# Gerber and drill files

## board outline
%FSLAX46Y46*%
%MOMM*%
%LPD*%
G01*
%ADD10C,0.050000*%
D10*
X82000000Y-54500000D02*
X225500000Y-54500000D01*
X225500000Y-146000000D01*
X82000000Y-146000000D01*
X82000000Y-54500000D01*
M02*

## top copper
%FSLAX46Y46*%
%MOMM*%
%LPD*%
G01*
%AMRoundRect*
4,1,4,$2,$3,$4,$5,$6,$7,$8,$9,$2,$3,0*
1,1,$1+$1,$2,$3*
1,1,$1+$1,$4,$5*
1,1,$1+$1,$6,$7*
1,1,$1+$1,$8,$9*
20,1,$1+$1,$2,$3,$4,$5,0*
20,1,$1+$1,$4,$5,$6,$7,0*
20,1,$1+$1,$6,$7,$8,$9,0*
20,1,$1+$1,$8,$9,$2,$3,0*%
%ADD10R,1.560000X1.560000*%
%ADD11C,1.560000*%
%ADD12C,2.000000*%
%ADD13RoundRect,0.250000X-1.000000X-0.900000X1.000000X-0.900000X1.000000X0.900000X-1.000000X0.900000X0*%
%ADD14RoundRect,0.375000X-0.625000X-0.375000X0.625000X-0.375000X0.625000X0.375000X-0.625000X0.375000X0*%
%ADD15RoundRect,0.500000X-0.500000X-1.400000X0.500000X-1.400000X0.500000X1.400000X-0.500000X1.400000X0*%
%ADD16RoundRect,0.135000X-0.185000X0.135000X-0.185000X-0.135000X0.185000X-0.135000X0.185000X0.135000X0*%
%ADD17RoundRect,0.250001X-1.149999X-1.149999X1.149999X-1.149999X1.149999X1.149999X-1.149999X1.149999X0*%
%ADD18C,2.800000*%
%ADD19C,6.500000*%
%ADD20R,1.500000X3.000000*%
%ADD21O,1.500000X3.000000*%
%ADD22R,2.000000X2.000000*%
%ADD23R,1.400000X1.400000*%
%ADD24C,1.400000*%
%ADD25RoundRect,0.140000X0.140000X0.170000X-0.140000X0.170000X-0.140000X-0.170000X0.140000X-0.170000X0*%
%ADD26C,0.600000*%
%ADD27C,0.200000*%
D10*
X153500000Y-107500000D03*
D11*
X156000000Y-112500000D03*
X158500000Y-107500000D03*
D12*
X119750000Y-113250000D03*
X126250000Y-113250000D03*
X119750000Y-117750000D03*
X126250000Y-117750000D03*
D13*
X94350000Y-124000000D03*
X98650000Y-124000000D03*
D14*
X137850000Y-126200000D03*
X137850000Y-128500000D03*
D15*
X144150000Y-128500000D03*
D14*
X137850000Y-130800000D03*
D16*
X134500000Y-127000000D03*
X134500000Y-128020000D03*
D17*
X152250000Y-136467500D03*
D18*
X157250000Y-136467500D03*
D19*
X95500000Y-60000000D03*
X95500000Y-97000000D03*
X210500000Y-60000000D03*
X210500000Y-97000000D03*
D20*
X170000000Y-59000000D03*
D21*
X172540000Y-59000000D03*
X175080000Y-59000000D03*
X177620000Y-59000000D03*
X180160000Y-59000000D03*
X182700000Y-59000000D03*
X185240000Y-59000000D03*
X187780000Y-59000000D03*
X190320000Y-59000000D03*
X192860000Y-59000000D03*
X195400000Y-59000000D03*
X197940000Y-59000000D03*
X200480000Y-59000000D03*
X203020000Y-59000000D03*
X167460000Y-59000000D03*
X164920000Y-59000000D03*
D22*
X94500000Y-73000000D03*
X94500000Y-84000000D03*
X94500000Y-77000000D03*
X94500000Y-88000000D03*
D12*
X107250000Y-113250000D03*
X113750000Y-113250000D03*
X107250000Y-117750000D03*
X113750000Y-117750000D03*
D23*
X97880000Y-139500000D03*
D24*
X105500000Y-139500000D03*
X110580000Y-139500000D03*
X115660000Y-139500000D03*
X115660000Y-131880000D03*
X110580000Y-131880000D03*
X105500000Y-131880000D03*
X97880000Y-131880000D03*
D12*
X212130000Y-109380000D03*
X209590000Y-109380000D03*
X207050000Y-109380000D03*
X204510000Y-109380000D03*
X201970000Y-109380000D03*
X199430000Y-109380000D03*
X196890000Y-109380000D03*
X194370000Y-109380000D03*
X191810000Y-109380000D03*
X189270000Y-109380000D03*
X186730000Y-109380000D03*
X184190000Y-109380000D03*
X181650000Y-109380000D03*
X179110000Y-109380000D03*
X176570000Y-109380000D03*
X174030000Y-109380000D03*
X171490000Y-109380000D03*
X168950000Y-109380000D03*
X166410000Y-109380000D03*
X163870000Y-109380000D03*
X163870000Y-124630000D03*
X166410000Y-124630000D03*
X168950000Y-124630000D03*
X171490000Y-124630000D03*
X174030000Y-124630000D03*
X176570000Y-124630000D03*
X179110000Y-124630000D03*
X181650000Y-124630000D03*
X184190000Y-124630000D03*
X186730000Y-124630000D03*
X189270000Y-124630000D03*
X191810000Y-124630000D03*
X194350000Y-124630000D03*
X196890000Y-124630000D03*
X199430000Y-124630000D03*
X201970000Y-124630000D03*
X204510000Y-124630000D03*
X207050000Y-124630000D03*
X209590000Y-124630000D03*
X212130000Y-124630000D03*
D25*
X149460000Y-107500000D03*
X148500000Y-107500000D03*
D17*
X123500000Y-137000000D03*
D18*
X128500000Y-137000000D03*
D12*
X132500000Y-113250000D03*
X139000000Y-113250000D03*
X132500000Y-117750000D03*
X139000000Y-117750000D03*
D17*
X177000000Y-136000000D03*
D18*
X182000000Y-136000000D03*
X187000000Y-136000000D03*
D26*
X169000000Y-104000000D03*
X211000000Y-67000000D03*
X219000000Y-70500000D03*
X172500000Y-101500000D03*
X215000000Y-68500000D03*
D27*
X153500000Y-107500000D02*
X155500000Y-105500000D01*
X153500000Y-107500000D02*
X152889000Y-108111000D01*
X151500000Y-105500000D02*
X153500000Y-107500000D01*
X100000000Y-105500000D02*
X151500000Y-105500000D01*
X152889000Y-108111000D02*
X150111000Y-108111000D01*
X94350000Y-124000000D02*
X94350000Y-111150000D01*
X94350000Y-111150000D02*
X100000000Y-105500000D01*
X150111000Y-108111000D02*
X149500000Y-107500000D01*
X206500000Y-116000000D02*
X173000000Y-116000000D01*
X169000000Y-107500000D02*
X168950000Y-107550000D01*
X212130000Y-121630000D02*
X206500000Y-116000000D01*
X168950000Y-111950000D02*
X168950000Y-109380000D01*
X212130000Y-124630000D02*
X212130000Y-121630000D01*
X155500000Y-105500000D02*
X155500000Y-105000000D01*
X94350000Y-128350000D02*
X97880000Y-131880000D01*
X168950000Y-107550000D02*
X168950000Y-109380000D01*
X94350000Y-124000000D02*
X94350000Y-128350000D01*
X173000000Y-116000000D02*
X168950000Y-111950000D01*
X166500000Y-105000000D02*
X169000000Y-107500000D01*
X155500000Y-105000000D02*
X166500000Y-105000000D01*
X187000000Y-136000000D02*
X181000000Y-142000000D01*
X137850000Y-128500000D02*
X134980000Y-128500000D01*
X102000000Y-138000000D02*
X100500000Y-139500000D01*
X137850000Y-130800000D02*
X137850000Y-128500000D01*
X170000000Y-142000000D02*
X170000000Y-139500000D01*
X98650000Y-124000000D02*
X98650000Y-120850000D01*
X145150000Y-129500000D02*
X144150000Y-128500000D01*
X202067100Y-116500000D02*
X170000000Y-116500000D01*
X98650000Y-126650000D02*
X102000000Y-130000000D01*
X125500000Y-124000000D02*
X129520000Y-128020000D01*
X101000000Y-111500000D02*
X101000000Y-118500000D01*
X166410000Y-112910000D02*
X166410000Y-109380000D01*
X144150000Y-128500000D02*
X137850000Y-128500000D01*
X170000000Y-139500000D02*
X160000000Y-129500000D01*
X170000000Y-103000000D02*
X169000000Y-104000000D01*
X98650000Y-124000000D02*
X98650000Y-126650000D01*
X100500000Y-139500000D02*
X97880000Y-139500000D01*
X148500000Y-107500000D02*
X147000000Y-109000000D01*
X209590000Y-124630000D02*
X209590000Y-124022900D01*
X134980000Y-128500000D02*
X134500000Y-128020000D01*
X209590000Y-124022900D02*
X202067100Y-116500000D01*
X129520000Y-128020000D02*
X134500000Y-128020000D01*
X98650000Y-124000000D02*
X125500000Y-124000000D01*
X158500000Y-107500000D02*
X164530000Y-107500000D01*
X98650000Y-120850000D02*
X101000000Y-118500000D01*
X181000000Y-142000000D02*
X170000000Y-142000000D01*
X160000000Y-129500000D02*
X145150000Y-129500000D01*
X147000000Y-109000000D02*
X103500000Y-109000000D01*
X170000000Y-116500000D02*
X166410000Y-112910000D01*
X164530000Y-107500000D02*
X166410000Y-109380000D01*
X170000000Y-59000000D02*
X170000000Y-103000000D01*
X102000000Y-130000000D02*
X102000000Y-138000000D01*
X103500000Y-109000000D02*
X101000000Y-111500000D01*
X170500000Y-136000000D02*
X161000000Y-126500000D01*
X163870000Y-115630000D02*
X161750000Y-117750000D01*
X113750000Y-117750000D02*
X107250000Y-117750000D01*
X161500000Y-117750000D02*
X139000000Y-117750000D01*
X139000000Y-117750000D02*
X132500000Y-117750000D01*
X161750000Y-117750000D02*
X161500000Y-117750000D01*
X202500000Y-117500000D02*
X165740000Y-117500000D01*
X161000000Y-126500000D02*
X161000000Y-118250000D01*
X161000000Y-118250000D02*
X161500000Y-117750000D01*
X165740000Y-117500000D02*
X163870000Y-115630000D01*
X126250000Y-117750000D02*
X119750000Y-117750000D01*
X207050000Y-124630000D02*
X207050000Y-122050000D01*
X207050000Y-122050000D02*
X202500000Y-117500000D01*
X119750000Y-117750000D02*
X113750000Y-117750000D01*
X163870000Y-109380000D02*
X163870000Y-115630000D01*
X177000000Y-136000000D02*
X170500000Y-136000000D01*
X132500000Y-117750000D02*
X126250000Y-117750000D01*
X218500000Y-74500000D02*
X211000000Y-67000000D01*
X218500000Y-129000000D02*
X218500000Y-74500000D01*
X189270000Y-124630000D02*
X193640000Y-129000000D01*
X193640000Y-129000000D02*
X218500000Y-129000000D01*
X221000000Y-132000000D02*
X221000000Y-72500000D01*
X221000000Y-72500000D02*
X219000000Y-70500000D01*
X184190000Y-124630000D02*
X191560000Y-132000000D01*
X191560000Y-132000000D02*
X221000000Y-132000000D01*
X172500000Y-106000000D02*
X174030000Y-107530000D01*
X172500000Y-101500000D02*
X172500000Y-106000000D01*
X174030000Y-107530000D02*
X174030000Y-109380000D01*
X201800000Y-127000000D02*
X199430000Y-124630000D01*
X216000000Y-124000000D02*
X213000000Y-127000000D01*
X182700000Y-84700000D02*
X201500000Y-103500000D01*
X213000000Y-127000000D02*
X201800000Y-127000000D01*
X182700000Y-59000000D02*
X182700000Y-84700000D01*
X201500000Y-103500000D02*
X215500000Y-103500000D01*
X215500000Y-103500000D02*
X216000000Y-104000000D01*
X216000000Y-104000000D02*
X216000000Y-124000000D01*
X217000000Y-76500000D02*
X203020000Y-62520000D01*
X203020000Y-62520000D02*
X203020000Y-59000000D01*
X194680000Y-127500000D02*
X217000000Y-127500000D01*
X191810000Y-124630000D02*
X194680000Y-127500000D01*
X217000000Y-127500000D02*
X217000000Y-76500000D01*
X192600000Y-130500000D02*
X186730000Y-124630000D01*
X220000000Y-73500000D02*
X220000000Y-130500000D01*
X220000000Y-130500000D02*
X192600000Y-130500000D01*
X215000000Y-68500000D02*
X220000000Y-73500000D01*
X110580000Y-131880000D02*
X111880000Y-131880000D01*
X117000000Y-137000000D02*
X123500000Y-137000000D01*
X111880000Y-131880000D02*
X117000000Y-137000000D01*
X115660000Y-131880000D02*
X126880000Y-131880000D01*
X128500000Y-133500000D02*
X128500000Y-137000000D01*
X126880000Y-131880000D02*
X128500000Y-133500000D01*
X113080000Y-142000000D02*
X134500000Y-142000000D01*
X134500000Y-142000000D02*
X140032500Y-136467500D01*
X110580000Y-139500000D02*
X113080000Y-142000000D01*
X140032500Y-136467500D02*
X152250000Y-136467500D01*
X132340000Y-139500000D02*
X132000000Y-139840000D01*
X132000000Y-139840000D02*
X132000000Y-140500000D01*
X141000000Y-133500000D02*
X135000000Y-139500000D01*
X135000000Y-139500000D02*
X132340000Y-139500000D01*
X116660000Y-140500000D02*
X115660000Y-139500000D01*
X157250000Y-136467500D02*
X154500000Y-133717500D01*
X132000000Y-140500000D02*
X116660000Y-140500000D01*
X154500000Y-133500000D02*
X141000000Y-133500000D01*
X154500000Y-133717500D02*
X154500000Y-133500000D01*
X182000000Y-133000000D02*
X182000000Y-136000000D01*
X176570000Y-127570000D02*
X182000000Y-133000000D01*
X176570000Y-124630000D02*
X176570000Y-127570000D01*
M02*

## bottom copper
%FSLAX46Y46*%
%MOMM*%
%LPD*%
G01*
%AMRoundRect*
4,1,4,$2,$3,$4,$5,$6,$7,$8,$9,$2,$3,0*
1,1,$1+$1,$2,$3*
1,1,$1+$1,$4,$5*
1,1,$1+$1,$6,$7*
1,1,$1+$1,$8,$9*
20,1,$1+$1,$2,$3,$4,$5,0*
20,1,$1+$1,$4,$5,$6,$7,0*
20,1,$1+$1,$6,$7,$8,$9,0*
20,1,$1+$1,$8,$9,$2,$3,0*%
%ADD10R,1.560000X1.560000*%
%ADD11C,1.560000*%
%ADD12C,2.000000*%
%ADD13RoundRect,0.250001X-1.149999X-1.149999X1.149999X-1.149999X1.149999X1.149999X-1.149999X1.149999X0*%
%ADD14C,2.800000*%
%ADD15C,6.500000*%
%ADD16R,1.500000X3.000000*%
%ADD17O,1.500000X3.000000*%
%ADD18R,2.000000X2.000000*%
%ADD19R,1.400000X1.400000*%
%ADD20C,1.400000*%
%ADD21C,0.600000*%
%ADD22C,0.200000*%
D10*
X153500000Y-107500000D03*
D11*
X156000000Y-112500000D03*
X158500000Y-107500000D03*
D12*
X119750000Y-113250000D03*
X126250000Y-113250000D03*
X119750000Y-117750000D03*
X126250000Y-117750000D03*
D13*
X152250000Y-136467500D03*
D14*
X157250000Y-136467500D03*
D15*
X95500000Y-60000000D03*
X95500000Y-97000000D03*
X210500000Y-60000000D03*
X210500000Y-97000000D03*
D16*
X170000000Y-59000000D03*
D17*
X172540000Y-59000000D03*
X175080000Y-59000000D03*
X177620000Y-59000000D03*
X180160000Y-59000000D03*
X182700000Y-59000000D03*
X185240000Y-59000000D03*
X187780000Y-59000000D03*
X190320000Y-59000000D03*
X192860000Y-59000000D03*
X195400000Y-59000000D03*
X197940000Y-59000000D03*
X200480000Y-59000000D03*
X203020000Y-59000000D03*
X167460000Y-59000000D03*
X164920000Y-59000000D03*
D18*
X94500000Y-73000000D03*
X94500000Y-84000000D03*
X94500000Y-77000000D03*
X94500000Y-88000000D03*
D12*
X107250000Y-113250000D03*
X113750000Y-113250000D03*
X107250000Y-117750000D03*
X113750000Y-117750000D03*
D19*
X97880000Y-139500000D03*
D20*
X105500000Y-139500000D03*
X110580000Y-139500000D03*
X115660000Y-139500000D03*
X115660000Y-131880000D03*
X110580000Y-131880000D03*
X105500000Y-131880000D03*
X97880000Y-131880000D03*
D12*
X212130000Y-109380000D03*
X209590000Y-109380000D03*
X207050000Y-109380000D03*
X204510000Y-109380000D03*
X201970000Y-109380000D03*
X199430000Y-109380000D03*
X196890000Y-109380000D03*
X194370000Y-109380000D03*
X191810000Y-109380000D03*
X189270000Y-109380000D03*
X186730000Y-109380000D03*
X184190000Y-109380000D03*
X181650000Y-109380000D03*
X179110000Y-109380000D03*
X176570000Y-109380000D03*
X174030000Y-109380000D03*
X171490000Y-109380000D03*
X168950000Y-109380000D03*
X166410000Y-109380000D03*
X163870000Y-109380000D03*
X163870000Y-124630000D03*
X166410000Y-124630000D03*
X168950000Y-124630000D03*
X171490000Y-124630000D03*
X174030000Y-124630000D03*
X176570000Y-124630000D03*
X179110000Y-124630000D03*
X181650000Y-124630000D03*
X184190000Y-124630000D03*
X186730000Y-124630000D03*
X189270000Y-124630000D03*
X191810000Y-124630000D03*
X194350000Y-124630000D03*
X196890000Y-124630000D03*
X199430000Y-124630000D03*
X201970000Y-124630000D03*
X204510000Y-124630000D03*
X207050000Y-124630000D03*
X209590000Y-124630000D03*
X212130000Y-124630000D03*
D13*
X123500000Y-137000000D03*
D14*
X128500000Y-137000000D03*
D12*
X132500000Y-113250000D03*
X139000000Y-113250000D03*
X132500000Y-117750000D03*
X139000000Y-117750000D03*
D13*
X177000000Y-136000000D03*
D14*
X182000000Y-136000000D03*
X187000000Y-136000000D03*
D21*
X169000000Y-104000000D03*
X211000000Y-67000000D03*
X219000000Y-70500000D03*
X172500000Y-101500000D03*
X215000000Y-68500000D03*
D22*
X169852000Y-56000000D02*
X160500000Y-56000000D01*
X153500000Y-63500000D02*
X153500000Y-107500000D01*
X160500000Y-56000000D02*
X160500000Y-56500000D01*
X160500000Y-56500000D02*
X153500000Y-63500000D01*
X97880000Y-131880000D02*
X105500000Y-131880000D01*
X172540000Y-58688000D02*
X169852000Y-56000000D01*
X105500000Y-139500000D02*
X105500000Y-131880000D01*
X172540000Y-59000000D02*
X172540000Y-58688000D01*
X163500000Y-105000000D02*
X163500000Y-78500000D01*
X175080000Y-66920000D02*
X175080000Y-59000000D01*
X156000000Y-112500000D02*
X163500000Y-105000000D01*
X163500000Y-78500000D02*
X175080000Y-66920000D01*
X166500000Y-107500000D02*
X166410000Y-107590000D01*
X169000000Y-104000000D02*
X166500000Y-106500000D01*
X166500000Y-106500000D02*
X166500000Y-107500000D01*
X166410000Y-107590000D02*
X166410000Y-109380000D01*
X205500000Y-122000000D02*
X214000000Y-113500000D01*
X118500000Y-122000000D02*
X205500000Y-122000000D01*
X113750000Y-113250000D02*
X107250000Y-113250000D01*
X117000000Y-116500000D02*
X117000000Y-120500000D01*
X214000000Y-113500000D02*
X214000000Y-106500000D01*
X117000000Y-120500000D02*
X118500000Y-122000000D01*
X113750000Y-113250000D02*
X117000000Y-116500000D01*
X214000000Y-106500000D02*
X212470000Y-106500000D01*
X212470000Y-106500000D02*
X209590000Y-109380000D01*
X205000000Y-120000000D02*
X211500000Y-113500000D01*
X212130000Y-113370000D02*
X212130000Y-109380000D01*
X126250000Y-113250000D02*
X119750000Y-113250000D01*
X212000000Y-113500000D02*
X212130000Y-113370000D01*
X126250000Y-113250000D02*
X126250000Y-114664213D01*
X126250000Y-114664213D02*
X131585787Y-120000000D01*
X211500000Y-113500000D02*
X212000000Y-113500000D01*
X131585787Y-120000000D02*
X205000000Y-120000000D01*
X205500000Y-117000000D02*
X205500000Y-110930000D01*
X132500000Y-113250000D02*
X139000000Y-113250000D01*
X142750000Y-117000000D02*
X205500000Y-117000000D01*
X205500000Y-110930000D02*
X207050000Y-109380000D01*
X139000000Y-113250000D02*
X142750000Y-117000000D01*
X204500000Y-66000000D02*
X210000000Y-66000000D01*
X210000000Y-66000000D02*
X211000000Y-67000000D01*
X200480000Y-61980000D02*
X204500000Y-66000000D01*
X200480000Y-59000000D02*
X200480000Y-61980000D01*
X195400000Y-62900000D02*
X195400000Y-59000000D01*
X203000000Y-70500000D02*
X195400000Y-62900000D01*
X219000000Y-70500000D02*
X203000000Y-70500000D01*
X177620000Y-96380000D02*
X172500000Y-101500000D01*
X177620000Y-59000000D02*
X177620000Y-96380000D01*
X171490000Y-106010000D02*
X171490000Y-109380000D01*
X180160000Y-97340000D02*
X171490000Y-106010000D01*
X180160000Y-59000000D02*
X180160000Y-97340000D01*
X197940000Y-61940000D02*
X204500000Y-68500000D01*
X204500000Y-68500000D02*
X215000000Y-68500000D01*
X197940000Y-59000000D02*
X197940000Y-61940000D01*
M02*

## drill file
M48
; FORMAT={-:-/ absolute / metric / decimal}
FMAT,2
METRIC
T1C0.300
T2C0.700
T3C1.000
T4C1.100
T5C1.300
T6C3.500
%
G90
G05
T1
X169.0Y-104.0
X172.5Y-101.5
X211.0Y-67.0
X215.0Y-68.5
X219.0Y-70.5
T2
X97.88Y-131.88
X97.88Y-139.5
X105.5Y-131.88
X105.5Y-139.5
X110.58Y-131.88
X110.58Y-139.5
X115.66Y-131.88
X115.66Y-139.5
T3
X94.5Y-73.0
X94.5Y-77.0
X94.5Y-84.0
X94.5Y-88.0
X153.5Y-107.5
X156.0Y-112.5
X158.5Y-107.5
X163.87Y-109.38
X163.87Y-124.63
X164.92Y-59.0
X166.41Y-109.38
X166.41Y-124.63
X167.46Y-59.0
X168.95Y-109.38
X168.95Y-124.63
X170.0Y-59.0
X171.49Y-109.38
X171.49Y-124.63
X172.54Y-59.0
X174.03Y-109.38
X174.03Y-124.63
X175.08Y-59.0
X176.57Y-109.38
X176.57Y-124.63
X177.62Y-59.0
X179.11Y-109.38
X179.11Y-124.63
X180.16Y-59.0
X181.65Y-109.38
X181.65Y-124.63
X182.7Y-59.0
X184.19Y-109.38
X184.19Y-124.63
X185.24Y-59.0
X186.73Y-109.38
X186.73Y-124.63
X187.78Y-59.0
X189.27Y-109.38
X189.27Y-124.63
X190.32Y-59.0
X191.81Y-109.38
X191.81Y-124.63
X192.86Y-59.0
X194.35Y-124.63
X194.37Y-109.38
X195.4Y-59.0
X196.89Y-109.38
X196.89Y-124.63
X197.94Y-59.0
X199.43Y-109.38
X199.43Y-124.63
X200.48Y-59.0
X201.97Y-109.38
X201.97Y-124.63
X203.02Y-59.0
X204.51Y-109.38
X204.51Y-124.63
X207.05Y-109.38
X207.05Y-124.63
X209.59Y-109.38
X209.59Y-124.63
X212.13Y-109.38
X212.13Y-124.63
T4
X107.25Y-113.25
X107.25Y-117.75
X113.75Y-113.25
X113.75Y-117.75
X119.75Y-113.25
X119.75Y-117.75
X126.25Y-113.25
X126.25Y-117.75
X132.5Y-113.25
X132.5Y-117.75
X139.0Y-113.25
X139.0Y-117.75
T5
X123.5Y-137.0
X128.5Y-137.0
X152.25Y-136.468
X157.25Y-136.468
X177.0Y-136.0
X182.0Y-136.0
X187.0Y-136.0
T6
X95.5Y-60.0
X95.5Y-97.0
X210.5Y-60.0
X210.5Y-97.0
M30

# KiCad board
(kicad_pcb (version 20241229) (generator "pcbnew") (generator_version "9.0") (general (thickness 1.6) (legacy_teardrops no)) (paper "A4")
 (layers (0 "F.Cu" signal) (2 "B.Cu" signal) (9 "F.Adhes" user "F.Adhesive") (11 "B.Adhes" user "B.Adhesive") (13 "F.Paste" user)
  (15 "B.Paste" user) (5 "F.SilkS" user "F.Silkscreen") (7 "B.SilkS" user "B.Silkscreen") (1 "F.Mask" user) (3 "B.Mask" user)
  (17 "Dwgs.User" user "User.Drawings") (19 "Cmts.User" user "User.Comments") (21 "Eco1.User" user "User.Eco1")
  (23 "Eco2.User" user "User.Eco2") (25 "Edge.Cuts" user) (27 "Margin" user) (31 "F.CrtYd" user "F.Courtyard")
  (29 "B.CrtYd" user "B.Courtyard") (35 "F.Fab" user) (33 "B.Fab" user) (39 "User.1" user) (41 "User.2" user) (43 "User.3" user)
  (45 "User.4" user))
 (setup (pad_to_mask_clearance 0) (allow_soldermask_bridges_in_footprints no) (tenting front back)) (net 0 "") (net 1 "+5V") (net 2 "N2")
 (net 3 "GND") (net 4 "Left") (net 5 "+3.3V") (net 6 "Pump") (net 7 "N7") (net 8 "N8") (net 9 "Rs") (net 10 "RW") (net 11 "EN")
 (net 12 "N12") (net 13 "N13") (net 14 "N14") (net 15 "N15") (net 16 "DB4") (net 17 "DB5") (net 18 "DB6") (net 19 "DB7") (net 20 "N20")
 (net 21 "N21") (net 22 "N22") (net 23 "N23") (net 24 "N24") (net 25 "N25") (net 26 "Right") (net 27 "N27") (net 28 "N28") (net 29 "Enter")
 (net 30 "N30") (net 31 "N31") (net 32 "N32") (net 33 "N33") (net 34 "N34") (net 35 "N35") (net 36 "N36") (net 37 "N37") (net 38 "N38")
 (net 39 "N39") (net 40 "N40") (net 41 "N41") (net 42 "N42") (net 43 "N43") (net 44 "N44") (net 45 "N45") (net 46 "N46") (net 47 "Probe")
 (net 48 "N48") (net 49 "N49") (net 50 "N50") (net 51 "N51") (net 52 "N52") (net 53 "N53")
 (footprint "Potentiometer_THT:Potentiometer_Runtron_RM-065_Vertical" (layer "F.Cu") (at 153.5 107.5)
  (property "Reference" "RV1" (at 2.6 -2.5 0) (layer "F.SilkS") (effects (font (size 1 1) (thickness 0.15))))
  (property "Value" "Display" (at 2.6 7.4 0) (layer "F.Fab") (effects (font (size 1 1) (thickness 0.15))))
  (pad "1" thru_hole rect (at 0 0) (size 1.56 1.56) (drill 1) (layers "*.Cu" "*.Mask") (remove_unused_layers no) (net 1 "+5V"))
  (pad "2" thru_hole circle (at 2.5 5) (size 1.56 1.56) (drill 1) (layers "*.Cu" "*.Mask") (remove_unused_layers no) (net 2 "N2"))
  (pad "3" thru_hole circle (at 5 0) (size 1.56 1.56) (drill 1) (layers "*.Cu" "*.Mask") (remove_unused_layers no) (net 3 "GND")))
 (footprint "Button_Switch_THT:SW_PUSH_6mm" (layer "F.Cu") (at 119.75 113.25)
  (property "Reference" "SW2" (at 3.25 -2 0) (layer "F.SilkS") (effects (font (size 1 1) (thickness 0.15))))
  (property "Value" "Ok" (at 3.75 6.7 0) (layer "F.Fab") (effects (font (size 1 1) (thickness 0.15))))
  (pad "1" thru_hole circle (at 0 0 90) (size 2 2) (drill 1.1) (layers "*.Cu" "*.Mask") (remove_unused_layers no) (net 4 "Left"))
  (pad "1" thru_hole circle (at 6.5 0 90) (size 2 2) (drill 1.1) (layers "*.Cu" "*.Mask") (remove_unused_layers no) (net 4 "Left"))
  (pad "2" thru_hole circle (at 0 4.5 90) (size 2 2) (drill 1.1) (layers "*.Cu" "*.Mask") (remove_unused_layers no) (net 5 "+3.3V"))
  (pad "2" thru_hole circle (at 6.5 4.5 90) (size 2 2) (drill 1.1) (layers "*.Cu" "*.Mask") (remove_unused_layers no) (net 5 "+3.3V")))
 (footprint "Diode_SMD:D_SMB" (layer "F.Cu") (at 96.5 124)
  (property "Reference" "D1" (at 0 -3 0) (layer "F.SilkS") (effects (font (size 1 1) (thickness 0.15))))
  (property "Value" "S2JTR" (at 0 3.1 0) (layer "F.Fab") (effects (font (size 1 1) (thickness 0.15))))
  (pad "1" smd roundrect (at -2.15 0) (size 2.5 2.3) (layers "F.Cu" "F.Mask" "F.Paste") (roundrect_rratio 0.1086956522) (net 1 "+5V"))
  (pad "2" smd roundrect (at 2.15 0) (size 2.5 2.3) (layers "F.Cu" "F.Mask" "F.Paste") (roundrect_rratio 0.1086956522) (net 3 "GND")))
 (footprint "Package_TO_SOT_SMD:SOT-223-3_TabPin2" (layer "F.Cu") (at 141 128.5)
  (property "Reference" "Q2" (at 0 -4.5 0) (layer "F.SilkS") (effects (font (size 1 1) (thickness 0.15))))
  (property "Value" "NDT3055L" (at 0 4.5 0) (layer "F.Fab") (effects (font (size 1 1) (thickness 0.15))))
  (pad "1" smd roundrect (at -3.15 -2.3) (size 2 1.5) (layers "F.Cu" "F.Mask" "F.Paste") (roundrect_rratio 0.25) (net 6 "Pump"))
  (pad "2" smd roundrect (at -3.15 0) (size 2 1.5) (layers "F.Cu" "F.Mask" "F.Paste") (roundrect_rratio 0.25) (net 3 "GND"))
  (pad "2" smd roundrect (at 3.15 0) (size 2 3.8) (layers "F.Cu" "F.Mask" "F.Paste") (roundrect_rratio 0.25) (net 3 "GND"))
  (pad "3" smd roundrect (at -3.15 2.3) (size 2 1.5) (layers "F.Cu" "F.Mask" "F.Paste") (roundrect_rratio 0.25) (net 3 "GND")))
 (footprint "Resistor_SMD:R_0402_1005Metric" (layer "F.Cu") (at 134.5 127.51 -90)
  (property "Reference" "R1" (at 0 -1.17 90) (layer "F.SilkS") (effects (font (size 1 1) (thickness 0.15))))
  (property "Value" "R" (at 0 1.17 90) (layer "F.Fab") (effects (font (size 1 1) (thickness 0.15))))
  (pad "1" smd roundrect (at -0.51 0 270) (size 0.54 0.64) (layers "F.Cu" "F.Mask" "F.Paste") (roundrect_rratio 0.25) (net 6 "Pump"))
  (pad "2" smd roundrect (at 0.51 0 270) (size 0.54 0.64) (layers "F.Cu" "F.Mask" "F.Paste") (roundrect_rratio 0.25) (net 3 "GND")))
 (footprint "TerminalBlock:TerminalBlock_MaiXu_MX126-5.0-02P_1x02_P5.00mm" (layer "F.Cu") (at 152.25 136.4675)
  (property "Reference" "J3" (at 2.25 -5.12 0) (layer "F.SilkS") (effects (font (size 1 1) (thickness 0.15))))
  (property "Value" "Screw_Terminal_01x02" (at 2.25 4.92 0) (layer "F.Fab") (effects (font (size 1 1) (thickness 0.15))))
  (pad "1" thru_hole roundrect (at 0 0) (size 2.8 2.8) (drill 1.3) (layers "*.Cu" "*.Mask") (remove_unused_layers no)
   (roundrect_rratio 0.089286) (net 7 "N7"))
  (pad "2" thru_hole circle (at 5 0) (size 2.8 2.8) (drill 1.3) (layers "*.Cu" "*.Mask") (remove_unused_layers no) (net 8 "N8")))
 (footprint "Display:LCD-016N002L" (layer "F.Cu") (at 170 59)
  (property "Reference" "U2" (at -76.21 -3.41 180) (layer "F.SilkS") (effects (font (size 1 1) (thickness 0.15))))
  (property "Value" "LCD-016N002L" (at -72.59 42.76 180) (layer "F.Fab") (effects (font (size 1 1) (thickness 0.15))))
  (pad "" thru_hole circle (at -74.5 1 180) (size 6.5 6.5) (drill 3.5) (layers "*.Cu" "*.Mask") (remove_unused_layers no))
  (pad "" thru_hole circle (at -74.5 38 180) (size 6.5 6.5) (drill 3.5) (layers "*.Cu" "*.Mask") (remove_unused_layers no))
  (pad "" thru_hole circle (at 40.5 1 180) (size 6.5 6.5) (drill 3.5) (layers "*.Cu" "*.Mask") (remove_unused_layers no))
  (pad "" thru_hole circle (at 40.5 38 180) (size 6.5 6.5) (drill 3.5) (layers "*.Cu" "*.Mask") (remove_unused_layers no))
  (pad "1" thru_hole rect (at 0 0 180) (size 1.5 3) (drill 1) (layers "*.Cu" "*.Mask") (remove_unused_layers no) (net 3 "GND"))
  (pad "2" thru_hole oval (at 2.54 0 180) (size 1.5 3) (drill 1) (layers "*.Cu" "*.Mask") (remove_unused_layers no) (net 1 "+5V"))
  (pad "3" thru_hole oval (at 5.08 0 180) (size 1.5 3) (drill 1) (layers "*.Cu" "*.Mask") (remove_unused_layers no) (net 2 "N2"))
  (pad "4" thru_hole oval (at 7.62 0 180) (size 1.5 3) (drill 1) (layers "*.Cu" "*.Mask") (remove_unused_layers no) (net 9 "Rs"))
  (pad "5" thru_hole oval (at 10.16 0 180) (size 1.5 3) (drill 1) (layers "*.Cu" "*.Mask") (remove_unused_layers no) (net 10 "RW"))
  (pad "6" thru_hole oval (at 12.7 0 180) (size 1.5 3) (drill 1) (layers "*.Cu" "*.Mask") (remove_unused_layers no) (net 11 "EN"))
  (pad "7" thru_hole oval (at 15.24 0 180) (size 1.5 3) (drill 1) (layers "*.Cu" "*.Mask") (remove_unused_layers no) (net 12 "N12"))
  (pad "8" thru_hole oval (at 17.78 0 180) (size 1.5 3) (drill 1) (layers "*.Cu" "*.Mask") (remove_unused_layers no) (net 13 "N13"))
  (pad "9" thru_hole oval (at 20.32 0 180) (size 1.5 3) (drill 1) (layers "*.Cu" "*.Mask") (remove_unused_layers no) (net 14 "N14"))
  (pad "10" thru_hole oval (at 22.86 0 180) (size 1.5 3) (drill 1) (layers "*.Cu" "*.Mask") (remove_unused_layers no) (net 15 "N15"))
  (pad "11" thru_hole oval (at 25.4 0 180) (size 1.5 3) (drill 1) (layers "*.Cu" "*.Mask") (remove_unused_layers no) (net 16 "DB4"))
  (pad "12" thru_hole oval (at 27.94 0 180) (size 1.5 3) (drill 1) (layers "*.Cu" "*.Mask") (remove_unused_layers no) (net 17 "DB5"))
  (pad "13" thru_hole oval (at 30.48 0 180) (size 1.5 3) (drill 1) (layers "*.Cu" "*.Mask") (remove_unused_layers no) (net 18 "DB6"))
  (pad "14" thru_hole oval (at 33.02 0 180) (size 1.5 3) (drill 1) (layers "*.Cu" "*.Mask") (remove_unused_layers no) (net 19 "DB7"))
  (pad "15" thru_hole oval (at -2.54 0 180) (size 1.5 3) (drill 1) (layers "*.Cu" "*.Mask") (remove_unused_layers no) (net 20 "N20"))
  (pad "16" thru_hole oval (at -5.08 0 180) (size 1.5 3) (drill 1) (layers "*.Cu" "*.Mask") (remove_unused_layers no) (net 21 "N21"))
  (pad "A1" thru_hole rect (at -75.5 14 180) (size 2 2) (drill 1) (layers "*.Cu" "*.Mask") (remove_unused_layers no) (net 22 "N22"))
  (pad "A2" thru_hole rect (at -75.5 25 180) (size 2 2) (drill 1) (layers "*.Cu" "*.Mask") (remove_unused_layers no) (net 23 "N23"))
  (pad "K1" thru_hole rect (at -75.5 18 180) (size 2 2) (drill 1) (layers "*.Cu" "*.Mask") (remove_unused_layers no) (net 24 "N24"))
  (pad "K2" thru_hole rect (at -75.5 29 180) (size 2 2) (drill 1) (layers "*.Cu" "*.Mask") (remove_unused_layers no) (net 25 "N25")))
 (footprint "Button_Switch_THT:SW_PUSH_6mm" (layer "F.Cu") (at 107.25 113.25)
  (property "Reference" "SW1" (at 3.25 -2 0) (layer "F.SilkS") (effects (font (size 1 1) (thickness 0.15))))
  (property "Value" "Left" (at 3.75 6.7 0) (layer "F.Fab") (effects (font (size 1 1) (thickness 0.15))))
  (pad "1" thru_hole circle (at 0 0 90) (size 2 2) (drill 1.1) (layers "*.Cu" "*.Mask") (remove_unused_layers no) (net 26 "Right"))
  (pad "1" thru_hole circle (at 6.5 0 90) (size 2 2) (drill 1.1) (layers "*.Cu" "*.Mask") (remove_unused_layers no) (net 26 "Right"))
  (pad "2" thru_hole circle (at 0 4.5 90) (size 2 2) (drill 1.1) (layers "*.Cu" "*.Mask") (remove_unused_layers no) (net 5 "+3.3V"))
  (pad "2" thru_hole circle (at 6.5 4.5 90) (size 2 2) (drill 1.1) (layers "*.Cu" "*.Mask") (remove_unused_layers no) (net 5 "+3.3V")))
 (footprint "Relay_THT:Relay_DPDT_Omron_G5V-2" (layer "F.Cu") (at 97.88 139.5 90)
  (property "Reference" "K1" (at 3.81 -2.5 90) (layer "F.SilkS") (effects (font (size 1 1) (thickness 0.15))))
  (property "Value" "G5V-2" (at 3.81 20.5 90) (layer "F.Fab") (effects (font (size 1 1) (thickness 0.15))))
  (pad "1" thru_hole rect (at 0 0 90) (size 1.4 1.4) (drill 0.7) (layers "*.Cu" "*.Mask") (remove_unused_layers no) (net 3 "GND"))
  (pad "4" thru_hole circle (at 0 7.62 90) (size 1.4 1.4) (drill 0.7) (layers "*.Cu" "*.Mask") (remove_unused_layers no) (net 1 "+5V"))
  (pad "6" thru_hole circle (at 0 12.7 90) (size 1.4 1.4) (drill 0.7) (layers "*.Cu" "*.Mask") (remove_unused_layers no) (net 7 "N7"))
  (pad "8" thru_hole circle (at 0 17.78 90) (size 1.4 1.4) (drill 0.7) (layers "*.Cu" "*.Mask") (remove_unused_layers no) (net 8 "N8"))
  (pad "9" thru_hole circle (at 7.62 17.78 90) (size 1.4 1.4) (drill 0.7) (layers "*.Cu" "*.Mask") (remove_unused_layers no) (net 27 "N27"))
  (pad "11" thru_hole circle (at 7.62 12.7 90) (size 1.4 1.4) (drill 0.7) (layers "*.Cu" "*.Mask") (remove_unused_layers no) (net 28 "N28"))
  (pad "13" thru_hole circle (at 7.62 7.62 90) (size 1.4 1.4) (drill 0.7) (layers "*.Cu" "*.Mask") (remove_unused_layers no) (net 1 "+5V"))
  (pad "16" thru_hole circle (at 7.62 0 90) (size 1.4 1.4) (drill 0.7) (layers "*.Cu" "*.Mask") (remove_unused_layers no) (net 1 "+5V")))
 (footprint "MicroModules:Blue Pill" (layer "F.Cu") (at 212.13 109.38 90)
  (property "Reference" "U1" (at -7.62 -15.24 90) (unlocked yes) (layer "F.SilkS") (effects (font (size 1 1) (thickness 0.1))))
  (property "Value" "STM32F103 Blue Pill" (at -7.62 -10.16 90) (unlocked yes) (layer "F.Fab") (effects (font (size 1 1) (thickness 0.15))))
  (pad "1" thru_hole circle (at 0 0 90) (size 2 2) (drill 1) (layers "*.Cu" "*.Mask") (remove_unused_layers no) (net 4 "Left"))
  (pad "2" thru_hole circle (at 0 -2.54 90) (size 2 2) (drill 1) (layers "*.Cu" "*.Mask") (remove_unused_layers no) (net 26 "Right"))
  (pad "3" thru_hole circle (at 0 -5.08 90) (size 2 2) (drill 1) (layers "*.Cu" "*.Mask") (remove_unused_layers no) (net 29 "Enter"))
  (pad "4" thru_hole circle (at 0 -7.62 90) (size 2 2) (drill 1) (layers "*.Cu" "*.Mask") (remove_unused_layers no) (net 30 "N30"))
  (pad "5" thru_hole circle (at 0 -10.16 90) (size 2 2) (drill 1) (layers "*.Cu" "*.Mask") (remove_unused_layers no) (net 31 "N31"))
  (pad "6" thru_hole circle (at 0 -12.7 90) (size 2 2) (drill 1) (layers "*.Cu" "*.Mask") (remove_unused_layers no) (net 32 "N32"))
  (pad "7" thru_hole circle (at 0 -15.24 90) (size 2 2) (drill 1) (layers "*.Cu" "*.Mask") (remove_unused_layers no) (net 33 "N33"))
  (pad "8" thru_hole circle (at 0 -17.76 90) (size 2 2) (drill 1) (layers "*.Cu" "*.Mask") (remove_unused_layers no) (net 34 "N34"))
  (pad "9" thru_hole circle (at 0 -20.32 90) (size 2 2) (drill 1) (layers "*.Cu" "*.Mask") (remove_unused_layers no) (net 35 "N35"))
  (pad "10" thru_hole circle (at 0 -22.86 90) (size 2 2) (drill 1) (layers "*.Cu" "*.Mask") (remove_unused_layers no) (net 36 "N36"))
  (pad "11" thru_hole circle (at 0 -25.4 90) (size 2 2) (drill 1) (layers "*.Cu" "*.Mask") (remove_unused_layers no) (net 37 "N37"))
  (pad "12" thru_hole circle (at 0 -27.94 90) (size 2 2) (drill 1) (layers "*.Cu" "*.Mask") (remove_unused_layers no) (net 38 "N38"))
  (pad "13" thru_hole circle (at 0 -30.48 90) (size 2 2) (drill 1) (layers "*.Cu" "*.Mask") (remove_unused_layers no) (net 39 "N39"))
  (pad "14" thru_hole circle (at 0 -33.02 90) (size 2 2) (drill 1) (layers "*.Cu" "*.Mask") (remove_unused_layers no) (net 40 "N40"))
  (pad "15" thru_hole circle (at 0 -35.56 90) (size 2 2) (drill 1) (layers "*.Cu" "*.Mask") (remove_unused_layers no) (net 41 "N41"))
  (pad "16" thru_hole circle (at 0 -38.1 90) (size 2 2) (drill 1) (layers "*.Cu" "*.Mask") (remove_unused_layers no) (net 9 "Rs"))
  (pad "17" thru_hole circle (at 0 -40.64 90) (size 2 2) (drill 1) (layers "*.Cu" "*.Mask") (remove_unused_layers no) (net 10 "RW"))
  (pad "18" thru_hole circle (at 0 -43.18 90) (size 2 2) (drill 1) (layers "*.Cu" "*.Mask") (remove_unused_layers no) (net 1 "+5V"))
  (pad "19" thru_hole circle (at 0 -45.72 90) (size 2 2) (drill 1) (layers "*.Cu" "*.Mask") (remove_unused_layers no) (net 3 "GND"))
  (pad "20" thru_hole circle (at 0 -48.26 90) (size 2 2) (drill 1) (layers "*.Cu" "*.Mask") (remove_unused_layers no) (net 5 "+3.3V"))
  (pad "21" thru_hole circle (at -15.25 -48.26 90) (size 2 2) (drill 1) (layers "*.Cu" "*.Mask") (remove_unused_layers no) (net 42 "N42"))
  (pad "22" thru_hole circle (at -15.25 -45.72 90) (size 2 2) (drill 1) (layers "*.Cu" "*.Mask") (remove_unused_layers no) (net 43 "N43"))
  (pad "23" thru_hole circle (at -15.25 -43.18 90) (size 2 2) (drill 1) (layers "*.Cu" "*.Mask") (remove_unused_layers no) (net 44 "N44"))
  (pad "24" thru_hole circle (at -15.25 -40.64 90) (size 2 2) (drill 1) (layers "*.Cu" "*.Mask") (remove_unused_layers no) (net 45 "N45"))
  (pad "25" thru_hole circle (at -15.25 -38.1 90) (size 2 2) (drill 1) (layers "*.Cu" "*.Mask") (remove_unused_layers no) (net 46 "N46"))
  (pad "26" thru_hole circle (at -15.25 -35.56 90) (size 2 2) (drill 1) (layers "*.Cu" "*.Mask") (remove_unused_layers no) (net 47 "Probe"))
  (pad "27" thru_hole circle (at -15.25 -33.02 90) (size 2 2) (drill 1) (layers "*.Cu" "*.Mask") (remove_unused_layers no) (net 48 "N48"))
  (pad "28" thru_hole circle (at -15.25 -30.48 90) (size 2 2) (drill 1) (layers "*.Cu" "*.Mask") (remove_unused_layers no) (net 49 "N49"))
  (pad "29" thru_hole circle (at -15.25 -27.94 90) (size 2 2) (drill 1) (layers "*.Cu" "*.Mask") (remove_unused_layers no) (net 16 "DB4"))
  (pad "30" thru_hole circle (at -15.25 -25.4 90) (size 2 2) (drill 1) (layers "*.Cu" "*.Mask") (remove_unused_layers no) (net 17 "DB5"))
  (pad "31" thru_hole circle (at -15.25 -22.86 90) (size 2 2) (drill 1) (layers "*.Cu" "*.Mask") (remove_unused_layers no) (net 18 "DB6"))
  (pad "32" thru_hole circle (at -15.25 -20.32 90) (size 2 2) (drill 1) (layers "*.Cu" "*.Mask") (remove_unused_layers no) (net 19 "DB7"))
  (pad "33" thru_hole circle (at -15.25 -17.78 90) (size 2 2) (drill 1) (layers "*.Cu" "*.Mask") (remove_unused_layers no) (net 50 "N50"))
  (pad "34" thru_hole circle (at -15.25 -15.24 90) (size 2 2) (drill 1) (layers "*.Cu" "*.Mask") (remove_unused_layers no) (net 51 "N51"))
  (pad "35" thru_hole circle (at -15.25 -12.7 90) (size 2 2) (drill 1) (layers "*.Cu" "*.Mask") (remove_unused_layers no) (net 11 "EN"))
  (pad "36" thru_hole circle (at -15.25 -10.16 90) (size 2 2) (drill 1) (layers "*.Cu" "*.Mask") (remove_unused_layers no) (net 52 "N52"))
  (pad "37" thru_hole circle (at -15.25 -7.62 90) (size 2 2) (drill 1) (layers "*.Cu" "*.Mask") (remove_unused_layers no) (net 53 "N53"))
  (pad "38" thru_hole circle (at -15.25 -5.08 90) (size 2 2) (drill 1) (layers "*.Cu" "*.Mask") (remove_unused_layers no) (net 5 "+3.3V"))
  (pad "39" thru_hole circle (at -15.25 -2.54 90) (size 2 2) (drill 1) (layers "*.Cu" "*.Mask") (remove_unused_layers no) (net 3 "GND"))
  (pad "40" thru_hole circle (at -15.25 0 90) (size 2 2) (drill 1) (layers "*.Cu" "*.Mask") (remove_unused_layers no) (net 1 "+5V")))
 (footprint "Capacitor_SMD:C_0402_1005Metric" (layer "F.Cu") (at 148.98 107.5 180)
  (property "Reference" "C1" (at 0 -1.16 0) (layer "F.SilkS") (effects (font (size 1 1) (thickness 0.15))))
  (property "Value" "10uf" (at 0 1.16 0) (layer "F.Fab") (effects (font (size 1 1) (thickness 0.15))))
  (pad "1" smd roundrect (at -0.48 0 180) (size 0.56 0.62) (layers "F.Cu" "F.Mask" "F.Paste") (roundrect_rratio 0.25) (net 1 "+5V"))
  (pad "2" smd roundrect (at 0.48 0 180) (size 0.56 0.62) (layers "F.Cu" "F.Mask" "F.Paste") (roundrect_rratio 0.25) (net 3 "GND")))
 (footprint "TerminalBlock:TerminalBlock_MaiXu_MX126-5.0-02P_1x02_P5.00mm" (layer "F.Cu") (at 123.5 137)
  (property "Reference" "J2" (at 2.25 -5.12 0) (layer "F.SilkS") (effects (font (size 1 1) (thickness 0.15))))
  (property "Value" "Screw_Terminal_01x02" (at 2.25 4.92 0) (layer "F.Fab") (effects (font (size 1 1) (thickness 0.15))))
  (pad "1" thru_hole roundrect (at 0 0) (size 2.8 2.8) (drill 1.3) (layers "*.Cu" "*.Mask") (remove_unused_layers no)
   (roundrect_rratio 0.089286) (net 28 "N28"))
  (pad "2" thru_hole circle (at 5 0) (size 2.8 2.8) (drill 1.3) (layers "*.Cu" "*.Mask") (remove_unused_layers no) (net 27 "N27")))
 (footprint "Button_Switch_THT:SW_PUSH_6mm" (layer "F.Cu") (at 132.5 113.25)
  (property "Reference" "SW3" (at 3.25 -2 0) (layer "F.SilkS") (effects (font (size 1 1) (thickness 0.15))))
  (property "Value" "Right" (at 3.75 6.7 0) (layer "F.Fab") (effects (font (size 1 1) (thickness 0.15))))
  (pad "1" thru_hole circle (at 0 0 90) (size 2 2) (drill 1.1) (layers "*.Cu" "*.Mask") (remove_unused_layers no) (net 29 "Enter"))
  (pad "1" thru_hole circle (at 6.5 0 90) (size 2 2) (drill 1.1) (layers "*.Cu" "*.Mask") (remove_unused_layers no) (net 29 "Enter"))
  (pad "2" thru_hole circle (at 0 4.5 90) (size 2 2) (drill 1.1) (layers "*.Cu" "*.Mask") (remove_unused_layers no) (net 5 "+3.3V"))
  (pad "2" thru_hole circle (at 6.5 4.5 90) (size 2 2) (drill 1.1) (layers "*.Cu" "*.Mask") (remove_unused_layers no) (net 5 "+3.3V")))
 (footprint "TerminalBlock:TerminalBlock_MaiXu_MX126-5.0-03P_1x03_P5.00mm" (layer "F.Cu") (at 177 136)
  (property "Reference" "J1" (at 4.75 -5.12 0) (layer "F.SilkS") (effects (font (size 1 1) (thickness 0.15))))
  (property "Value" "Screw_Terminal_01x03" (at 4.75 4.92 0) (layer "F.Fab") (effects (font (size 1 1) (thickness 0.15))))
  (pad "1" thru_hole roundrect (at 0 0) (size 2.8 2.8) (drill 1.3) (layers "*.Cu" "*.Mask") (remove_unused_layers no)
   (roundrect_rratio 0.089286) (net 5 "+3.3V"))
  (pad "2" thru_hole circle (at 5 0) (size 2.8 2.8) (drill 1.3) (layers "*.Cu" "*.Mask") (remove_unused_layers no) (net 47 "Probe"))
  (pad "3" thru_hole circle (at 10 0) (size 2.8 2.8) (drill 1.3) (layers "*.Cu" "*.Mask") (remove_unused_layers no) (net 3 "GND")))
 (gr_rect (start 82 54.5) (end 225.5 146) (stroke (width 0.05) (type default)) (fill no) (layer "Edge.Cuts"))
 (segment (start 153.5 107.5) (end 155.5 105.5) (width 0.2) (layer "F.Cu") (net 1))
 (segment (start 153.5 107.5) (end 152.889 108.111) (width 0.2) (layer "F.Cu") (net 1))
 (segment (start 151.5 105.5) (end 153.5 107.5) (width 0.2) (layer "F.Cu") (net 1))
 (segment (start 100 105.5) (end 151.5 105.5) (width 0.2) (layer "F.Cu") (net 1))
 (segment (start 152.889 108.111) (end 150.111 108.111) (width 0.2) (layer "F.Cu") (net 1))
 (segment (start 94.35 124) (end 94.35 111.15) (width 0.2) (layer "F.Cu") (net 1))
 (segment (start 94.35 111.15) (end 100 105.5) (width 0.2) (layer "F.Cu") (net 1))
 (segment (start 150.111 108.111) (end 149.5 107.5) (width 0.2) (layer "F.Cu") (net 1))
 (segment (start 206.5 116) (end 173 116) (width 0.2) (layer "F.Cu") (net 1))
 (segment (start 169 107.5) (end 168.95 107.55) (width 0.2) (layer "F.Cu") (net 1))
 (segment (start 212.13 121.63) (end 206.5 116) (width 0.2) (layer "F.Cu") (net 1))
 (segment (start 168.95 111.95) (end 168.95 109.38) (width 0.2) (layer "F.Cu") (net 1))
 (segment (start 212.13 124.63) (end 212.13 121.63) (width 0.2) (layer "F.Cu") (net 1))
 (segment (start 155.5 105.5) (end 155.5 105) (width 0.2) (layer "F.Cu") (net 1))
 (segment (start 94.35 128.35) (end 97.88 131.88) (width 0.2) (layer "F.Cu") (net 1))
 (segment (start 168.95 107.55) (end 168.95 109.38) (width 0.2) (layer "F.Cu") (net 1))
 (segment (start 94.35 124) (end 94.35 128.35) (width 0.2) (layer "F.Cu") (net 1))
 (segment (start 173 116) (end 168.95 111.95) (width 0.2) (layer "F.Cu") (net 1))
 (segment (start 166.5 105) (end 169 107.5) (width 0.2) (layer "F.Cu") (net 1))
 (segment (start 155.5 105) (end 166.5 105) (width 0.2) (layer "F.Cu") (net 1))
 (segment (start 169.852 56) (end 160.5 56) (width 0.2) (layer "B.Cu") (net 1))
 (segment (start 153.5 63.5) (end 153.5 107.5) (width 0.2) (layer "B.Cu") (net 1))
 (segment (start 160.5 56) (end 160.5 56.5) (width 0.2) (layer "B.Cu") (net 1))
 (segment (start 160.5 56.5) (end 153.5 63.5) (width 0.2) (layer "B.Cu") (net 1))
 (segment (start 97.88 131.88) (end 105.5 131.88) (width 0.2) (layer "B.Cu") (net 1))
 (segment (start 172.54 58.688) (end 169.852 56) (width 0.2) (layer "B.Cu") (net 1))
 (segment (start 105.5 139.5) (end 105.5 131.88) (width 0.2) (layer "B.Cu") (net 1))
 (segment (start 172.54 59) (end 172.54 58.688) (width 0.2) (layer "B.Cu") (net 1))
 (segment (start 163.5 105) (end 163.5 78.5) (width 0.2) (layer "B.Cu") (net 2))
 (segment (start 175.08 66.92) (end 175.08 59) (width 0.2) (layer "B.Cu") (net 2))
 (segment (start 156 112.5) (end 163.5 105) (width 0.2) (layer "B.Cu") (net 2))
 (segment (start 163.5 78.5) (end 175.08 66.92) (width 0.2) (layer "B.Cu") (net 2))
 (segment (start 187 136) (end 181 142) (width 0.2) (layer "F.Cu") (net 3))
 (segment (start 137.85 128.5) (end 134.98 128.5) (width 0.2) (layer "F.Cu") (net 3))
 (segment (start 102 138) (end 100.5 139.5) (width 0.2) (layer "F.Cu") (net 3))
 (segment (start 137.85 130.8) (end 137.85 128.5) (width 0.2) (layer "F.Cu") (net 3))
 (segment (start 170 142) (end 170 139.5) (width 0.2) (layer "F.Cu") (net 3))
 (segment (start 98.65 124) (end 98.65 120.85) (width 0.2) (layer "F.Cu") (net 3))
 (segment (start 145.15 129.5) (end 144.15 128.5) (width 0.2) (layer "F.Cu") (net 3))
 (segment (start 202.0671 116.5) (end 170 116.5) (width 0.2) (layer "F.Cu") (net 3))
 (segment (start 98.65 126.65) (end 102 130) (width 0.2) (layer "F.Cu") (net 3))
 (segment (start 125.5 124) (end 129.52 128.02) (width 0.2) (layer "F.Cu") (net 3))
 (segment (start 101 111.5) (end 101 118.5) (width 0.2) (layer "F.Cu") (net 3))
 (segment (start 166.41 112.91) (end 166.41 109.38) (width 0.2) (layer "F.Cu") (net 3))
 (segment (start 144.15 128.5) (end 137.85 128.5) (width 0.2) (layer "F.Cu") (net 3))
 (segment (start 170 139.5) (end 160 129.5) (width 0.2) (layer "F.Cu") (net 3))
 (segment (start 170 103) (end 169 104) (width 0.2) (layer "F.Cu") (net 3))
 (segment (start 98.65 124) (end 98.65 126.65) (width 0.2) (layer "F.Cu") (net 3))
 (segment (start 100.5 139.5) (end 97.88 139.5) (width 0.2) (layer "F.Cu") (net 3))
 (segment (start 148.5 107.5) (end 147 109) (width 0.2) (layer "F.Cu") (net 3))
 (segment (start 209.59 124.63) (end 209.59 124.0229) (width 0.2) (layer "F.Cu") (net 3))
 (segment (start 134.98 128.5) (end 134.5 128.02) (width 0.2) (layer "F.Cu") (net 3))
 (segment (start 209.59 124.0229) (end 202.0671 116.5) (width 0.2) (layer "F.Cu") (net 3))
 (segment (start 129.52 128.02) (end 134.5 128.02) (width 0.2) (layer "F.Cu") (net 3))
 (segment (start 98.65 124) (end 125.5 124) (width 0.2) (layer "F.Cu") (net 3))
 (segment (start 158.5 107.5) (end 164.53 107.5) (width 0.2) (layer "F.Cu") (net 3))
 (segment (start 98.65 120.85) (end 101 118.5) (width 0.2) (layer "F.Cu") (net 3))
 (segment (start 181 142) (end 170 142) (width 0.2) (layer "F.Cu") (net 3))
 (segment (start 160 129.5) (end 145.15 129.5) (width 0.2) (layer "F.Cu") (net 3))
 (segment (start 147 109) (end 103.5 109) (width 0.2) (layer "F.Cu") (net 3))
 (segment (start 170 116.5) (end 166.41 112.91) (width 0.2) (layer "F.Cu") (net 3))
 (segment (start 164.53 107.5) (end 166.41 109.38) (width 0.2) (layer "F.Cu") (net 3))
 (segment (start 170 59) (end 170 103) (width 0.2) (layer "F.Cu") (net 3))
 (segment (start 102 130) (end 102 138) (width 0.2) (layer "F.Cu") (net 3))
 (segment (start 103.5 109) (end 101 111.5) (width 0.2) (layer "F.Cu") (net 3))
 (via (at 169 104) (size 0.6) (drill 0.3) (layers "F.Cu" "B.Cu") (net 3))
 (segment (start 166.5 107.5) (end 166.41 107.59) (width 0.2) (layer "B.Cu") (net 3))
 (segment (start 169 104) (end 166.5 106.5) (width 0.2) (layer "B.Cu") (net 3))
 (segment (start 166.5 106.5) (end 166.5 107.5) (width 0.2) (layer "B.Cu") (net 3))
 (segment (start 166.41 107.59) (end 166.41 109.38) (width 0.2) (layer "B.Cu") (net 3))
 (segment (start 170.5 136) (end 161 126.5) (width 0.2) (layer "F.Cu") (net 5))
 (segment (start 163.87 115.63) (end 161.75 117.75) (width 0.2) (layer "F.Cu") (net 5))
 (segment (start 113.75 117.75) (end 107.25 117.75) (width 0.2) (layer "F.Cu") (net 5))
 (segment (start 161.5 117.75) (end 139 117.75) (width 0.2) (layer "F.Cu") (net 5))
 (segment (start 139 117.75) (end 132.5 117.75) (width 0.2) (layer "F.Cu") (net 5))
 (segment (start 161.75 117.75) (end 161.5 117.75) (width 0.2) (layer "F.Cu") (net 5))
 (segment (start 202.5 117.5) (end 165.74 117.5) (width 0.2) (layer "F.Cu") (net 5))
 (segment (start 161 126.5) (end 161 118.25) (width 0.2) (layer "F.Cu") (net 5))
 (segment (start 161 118.25) (end 161.5 117.75) (width 0.2) (layer "F.Cu") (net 5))
 (segment (start 165.74 117.5) (end 163.87 115.63) (width 0.2) (layer "F.Cu") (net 5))
 (segment (start 126.25 117.75) (end 119.75 117.75) (width 0.2) (layer "F.Cu") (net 5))
 (segment (start 207.05 124.63) (end 207.05 122.05) (width 0.2) (layer "F.Cu") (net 5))
 (segment (start 207.05 122.05) (end 202.5 117.5) (width 0.2) (layer "F.Cu") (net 5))
 (segment (start 119.75 117.75) (end 113.75 117.75) (width 0.2) (layer "F.Cu") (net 5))
 (segment (start 163.87 109.38) (end 163.87 115.63) (width 0.2) (layer "F.Cu") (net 5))
 (segment (start 177 136) (end 170.5 136) (width 0.2) (layer "F.Cu") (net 5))
 (segment (start 132.5 117.75) (end 126.25 117.75) (width 0.2) (layer "F.Cu") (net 5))
 (segment (start 205.5 122) (end 214 113.5) (width 0.2) (layer "B.Cu") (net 26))
 (segment (start 118.5 122) (end 205.5 122) (width 0.2) (layer "B.Cu") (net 26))
 (segment (start 113.75 113.25) (end 107.25 113.25) (width 0.2) (layer "B.Cu") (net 26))
 (segment (start 117 116.5) (end 117 120.5) (width 0.2) (layer "B.Cu") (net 26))
 (segment (start 214 113.5) (end 214 106.5) (width 0.2) (layer "B.Cu") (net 26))
 (segment (start 117 120.5) (end 118.5 122) (width 0.2) (layer "B.Cu") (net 26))
 (segment (start 113.75 113.25) (end 117 116.5) (width 0.2) (layer "B.Cu") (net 26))
 (segment (start 214 106.5) (end 212.47 106.5) (width 0.2) (layer "B.Cu") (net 26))
 (segment (start 212.47 106.5) (end 209.59 109.38) (width 0.2) (layer "B.Cu") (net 26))
 (segment (start 205 120) (end 211.5 113.5) (width 0.2) (layer "B.Cu") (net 4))
 (segment (start 212.13 113.37) (end 212.13 109.38) (width 0.2) (layer "B.Cu") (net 4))
 (segment (start 126.25 113.25) (end 119.75 113.25) (width 0.2) (layer "B.Cu") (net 4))
 (segment (start 212 113.5) (end 212.13 113.37) (width 0.2) (layer "B.Cu") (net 4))
 (segment (start 126.25 113.25) (end 126.25 114.664213) (width 0.2) (layer "B.Cu") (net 4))
 (segment (start 126.25 114.664213) (end 131.585787 120) (width 0.2) (layer "B.Cu") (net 4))
 (segment (start 211.5 113.5) (end 212 113.5) (width 0.2) (layer "B.Cu") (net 4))
 (segment (start 131.585787 120) (end 205 120) (width 0.2) (layer "B.Cu") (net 4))
 (segment (start 205.5 117) (end 205.5 110.93) (width 0.2) (layer "B.Cu") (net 29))
 (segment (start 132.5 113.25) (end 139 113.25) (width 0.2) (layer "B.Cu") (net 29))
 (segment (start 142.75 117) (end 205.5 117) (width 0.2) (layer "B.Cu") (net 29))
 (segment (start 205.5 110.93) (end 207.05 109.38) (width 0.2) (layer "B.Cu") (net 29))
 (segment (start 139 113.25) (end 142.75 117) (width 0.2) (layer "B.Cu") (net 29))
 (segment (start 218.5 74.5) (end 211 67) (width 0.2) (layer "F.Cu") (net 18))
 (segment (start 218.5 129) (end 218.5 74.5) (width 0.2) (layer "F.Cu") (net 18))
 (segment (start 189.27 124.63) (end 193.64 129) (width 0.2) (layer "F.Cu") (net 18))
 (segment (start 193.64 129) (end 218.5 129) (width 0.2) (layer "F.Cu") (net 18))
 (via (at 211 67) (size 0.6) (drill 0.3) (layers "F.Cu" "B.Cu") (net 18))
 (segment (start 204.5 66) (end 210 66) (width 0.2) (layer "B.Cu") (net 18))
 (segment (start 210 66) (end 211 67) (width 0.2) (layer "B.Cu") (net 18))
 (segment (start 200.48 61.98) (end 204.5 66) (width 0.2) (layer "B.Cu") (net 18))
 (segment (start 200.48 59) (end 200.48 61.98) (width 0.2) (layer "B.Cu") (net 18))
 (segment (start 221 132) (end 221 72.5) (width 0.2) (layer "F.Cu") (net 16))
 (segment (start 221 72.5) (end 219 70.5) (width 0.2) (layer "F.Cu") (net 16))
 (segment (start 184.19 124.63) (end 191.56 132) (width 0.2) (layer "F.Cu") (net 16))
 (segment (start 191.56 132) (end 221 132) (width 0.2) (layer "F.Cu") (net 16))
 (via (at 219 70.5) (size 0.6) (drill 0.3) (layers "F.Cu" "B.Cu") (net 16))
 (segment (start 195.4 62.9) (end 195.4 59) (width 0.2) (layer "B.Cu") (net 16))
 (segment (start 203 70.5) (end 195.4 62.9) (width 0.2) (layer "B.Cu") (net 16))
 (segment (start 219 70.5) (end 203 70.5) (width 0.2) (layer "B.Cu") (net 16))
 (segment (start 172.5 106) (end 174.03 107.53) (width 0.2) (layer "F.Cu") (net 9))
 (segment (start 172.5 101.5) (end 172.5 106) (width 0.2) (layer "F.Cu") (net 9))
 (segment (start 174.03 107.53) (end 174.03 109.38) (width 0.2) (layer "F.Cu") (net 9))
 (via (at 172.5 101.5) (size 0.6) (drill 0.3) (layers "F.Cu" "B.Cu") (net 9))
 (segment (start 177.62 96.38) (end 172.5 101.5) (width 0.2) (layer "B.Cu") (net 9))
 (segment (start 177.62 59) (end 177.62 96.38) (width 0.2) (layer "B.Cu") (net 9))
 (segment (start 201.8 127) (end 199.43 124.63) (width 0.2) (layer "F.Cu") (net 11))
 (segment (start 216 124) (end 213 127) (width 0.2) (layer "F.Cu") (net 11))
 (segment (start 182.7 84.7) (end 201.5 103.5) (width 0.2) (layer "F.Cu") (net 11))
 (segment (start 213 127) (end 201.8 127) (width 0.2) (layer "F.Cu") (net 11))
 (segment (start 182.7 59) (end 182.7 84.7) (width 0.2) (layer "F.Cu") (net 11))
 (segment (start 201.5 103.5) (end 215.5 103.5) (width 0.2) (layer "F.Cu") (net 11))
 (segment (start 215.5 103.5) (end 216 104) (width 0.2) (layer "F.Cu") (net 11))
 (segment (start 216 104) (end 216 124) (width 0.2) (layer "F.Cu") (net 11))
 (segment (start 217 76.5) (end 203.02 62.52) (width 0.2) (layer "F.Cu") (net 19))
 (segment (start 203.02 62.52) (end 203.02 59) (width 0.2) (layer "F.Cu") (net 19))
 (segment (start 194.68 127.5) (end 217 127.5) (width 0.2) (layer "F.Cu") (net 19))
 (segment (start 191.81 124.63) (end 194.68 127.5) (width 0.2) (layer "F.Cu") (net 19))
 (segment (start 217 127.5) (end 217 76.5) (width 0.2) (layer "F.Cu") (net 19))
 (segment (start 171.49 106.01) (end 171.49 109.38) (width 0.2) (layer "B.Cu") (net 10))
 (segment (start 180.16 97.34) (end 171.49 106.01) (width 0.2) (layer "B.Cu") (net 10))
 (segment (start 180.16 59) (end 180.16 97.34) (width 0.2) (layer "B.Cu") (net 10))
 (segment (start 192.6 130.5) (end 186.73 124.63) (width 0.2) (layer "F.Cu") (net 17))
 (segment (start 220 73.5) (end 220 130.5) (width 0.2) (layer "F.Cu") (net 17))
 (segment (start 220 130.5) (end 192.6 130.5) (width 0.2) (layer "F.Cu") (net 17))
 (segment (start 215 68.5) (end 220 73.5) (width 0.2) (layer "F.Cu") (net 17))
 (via (at 215 68.5) (size 0.6) (drill 0.3) (layers "F.Cu" "B.Cu") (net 17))
 (segment (start 197.94 61.94) (end 204.5 68.5) (width 0.2) (layer "B.Cu") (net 17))
 (segment (start 204.5 68.5) (end 215 68.5) (width 0.2) (layer "B.Cu") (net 17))
 (segment (start 197.94 59) (end 197.94 61.94) (width 0.2) (layer "B.Cu") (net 17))
 (segment (start 110.58 131.88) (end 111.88 131.88) (width 0.2) (layer "F.Cu") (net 28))
 (segment (start 117 137) (end 123.5 137) (width 0.2) (layer "F.Cu") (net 28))
 (segment (start 111.88 131.88) (end 117 137) (width 0.2) (layer "F.Cu") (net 28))
 (segment (start 115.66 131.88) (end 126.88 131.88) (width 0.2) (layer "F.Cu") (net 27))
 (segment (start 128.5 133.5) (end 128.5 137) (width 0.2) (layer "F.Cu") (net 27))
 (segment (start 126.88 131.88) (end 128.5 133.5) (width 0.2) (layer "F.Cu") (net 27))
 (segment (start 113.08 142) (end 134.5 142) (width 0.2) (layer "F.Cu") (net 7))
 (segment (start 134.5 142) (end 140.0325 136.4675) (width 0.2) (layer "F.Cu") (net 7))
 (segment (start 110.58 139.5) (end 113.08 142) (width 0.2) (layer "F.Cu") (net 7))
 (segment (start 140.0325 136.4675) (end 152.25 136.4675) (width 0.2) (layer "F.Cu") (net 7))
 (segment (start 132.34 139.5) (end 132 139.84) (width 0.2) (layer "F.Cu") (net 8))
 (segment (start 132 139.84) (end 132 140.5) (width 0.2) (layer "F.Cu") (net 8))
 (segment (start 141 133.5) (end 135 139.5) (width 0.2) (layer "F.Cu") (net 8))
 (segment (start 135 139.5) (end 132.34 139.5) (width 0.2) (layer "F.Cu") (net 8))
 (segment (start 116.66 140.5) (end 115.66 139.5) (width 0.2) (layer "F.Cu") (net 8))
 (segment (start 157.25 136.4675) (end 154.5 133.7175) (width 0.2) (layer "F.Cu") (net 8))
 (segment (start 132 140.5) (end 116.66 140.5) (width 0.2) (layer "F.Cu") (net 8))
 (segment (start 154.5 133.5) (end 141 133.5) (width 0.2) (layer "F.Cu") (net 8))
 (segment (start 154.5 133.7175) (end 154.5 133.5) (width 0.2) (layer "F.Cu") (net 8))
 (segment (start 182 133) (end 182 136) (width 0.2) (layer "F.Cu") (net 47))
 (segment (start 176.57 127.57) (end 182 133) (width 0.2) (layer "F.Cu") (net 47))
 (segment (start 176.57 124.63) (end 176.57 127.57) (width 0.2) (layer "F.Cu") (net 47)))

